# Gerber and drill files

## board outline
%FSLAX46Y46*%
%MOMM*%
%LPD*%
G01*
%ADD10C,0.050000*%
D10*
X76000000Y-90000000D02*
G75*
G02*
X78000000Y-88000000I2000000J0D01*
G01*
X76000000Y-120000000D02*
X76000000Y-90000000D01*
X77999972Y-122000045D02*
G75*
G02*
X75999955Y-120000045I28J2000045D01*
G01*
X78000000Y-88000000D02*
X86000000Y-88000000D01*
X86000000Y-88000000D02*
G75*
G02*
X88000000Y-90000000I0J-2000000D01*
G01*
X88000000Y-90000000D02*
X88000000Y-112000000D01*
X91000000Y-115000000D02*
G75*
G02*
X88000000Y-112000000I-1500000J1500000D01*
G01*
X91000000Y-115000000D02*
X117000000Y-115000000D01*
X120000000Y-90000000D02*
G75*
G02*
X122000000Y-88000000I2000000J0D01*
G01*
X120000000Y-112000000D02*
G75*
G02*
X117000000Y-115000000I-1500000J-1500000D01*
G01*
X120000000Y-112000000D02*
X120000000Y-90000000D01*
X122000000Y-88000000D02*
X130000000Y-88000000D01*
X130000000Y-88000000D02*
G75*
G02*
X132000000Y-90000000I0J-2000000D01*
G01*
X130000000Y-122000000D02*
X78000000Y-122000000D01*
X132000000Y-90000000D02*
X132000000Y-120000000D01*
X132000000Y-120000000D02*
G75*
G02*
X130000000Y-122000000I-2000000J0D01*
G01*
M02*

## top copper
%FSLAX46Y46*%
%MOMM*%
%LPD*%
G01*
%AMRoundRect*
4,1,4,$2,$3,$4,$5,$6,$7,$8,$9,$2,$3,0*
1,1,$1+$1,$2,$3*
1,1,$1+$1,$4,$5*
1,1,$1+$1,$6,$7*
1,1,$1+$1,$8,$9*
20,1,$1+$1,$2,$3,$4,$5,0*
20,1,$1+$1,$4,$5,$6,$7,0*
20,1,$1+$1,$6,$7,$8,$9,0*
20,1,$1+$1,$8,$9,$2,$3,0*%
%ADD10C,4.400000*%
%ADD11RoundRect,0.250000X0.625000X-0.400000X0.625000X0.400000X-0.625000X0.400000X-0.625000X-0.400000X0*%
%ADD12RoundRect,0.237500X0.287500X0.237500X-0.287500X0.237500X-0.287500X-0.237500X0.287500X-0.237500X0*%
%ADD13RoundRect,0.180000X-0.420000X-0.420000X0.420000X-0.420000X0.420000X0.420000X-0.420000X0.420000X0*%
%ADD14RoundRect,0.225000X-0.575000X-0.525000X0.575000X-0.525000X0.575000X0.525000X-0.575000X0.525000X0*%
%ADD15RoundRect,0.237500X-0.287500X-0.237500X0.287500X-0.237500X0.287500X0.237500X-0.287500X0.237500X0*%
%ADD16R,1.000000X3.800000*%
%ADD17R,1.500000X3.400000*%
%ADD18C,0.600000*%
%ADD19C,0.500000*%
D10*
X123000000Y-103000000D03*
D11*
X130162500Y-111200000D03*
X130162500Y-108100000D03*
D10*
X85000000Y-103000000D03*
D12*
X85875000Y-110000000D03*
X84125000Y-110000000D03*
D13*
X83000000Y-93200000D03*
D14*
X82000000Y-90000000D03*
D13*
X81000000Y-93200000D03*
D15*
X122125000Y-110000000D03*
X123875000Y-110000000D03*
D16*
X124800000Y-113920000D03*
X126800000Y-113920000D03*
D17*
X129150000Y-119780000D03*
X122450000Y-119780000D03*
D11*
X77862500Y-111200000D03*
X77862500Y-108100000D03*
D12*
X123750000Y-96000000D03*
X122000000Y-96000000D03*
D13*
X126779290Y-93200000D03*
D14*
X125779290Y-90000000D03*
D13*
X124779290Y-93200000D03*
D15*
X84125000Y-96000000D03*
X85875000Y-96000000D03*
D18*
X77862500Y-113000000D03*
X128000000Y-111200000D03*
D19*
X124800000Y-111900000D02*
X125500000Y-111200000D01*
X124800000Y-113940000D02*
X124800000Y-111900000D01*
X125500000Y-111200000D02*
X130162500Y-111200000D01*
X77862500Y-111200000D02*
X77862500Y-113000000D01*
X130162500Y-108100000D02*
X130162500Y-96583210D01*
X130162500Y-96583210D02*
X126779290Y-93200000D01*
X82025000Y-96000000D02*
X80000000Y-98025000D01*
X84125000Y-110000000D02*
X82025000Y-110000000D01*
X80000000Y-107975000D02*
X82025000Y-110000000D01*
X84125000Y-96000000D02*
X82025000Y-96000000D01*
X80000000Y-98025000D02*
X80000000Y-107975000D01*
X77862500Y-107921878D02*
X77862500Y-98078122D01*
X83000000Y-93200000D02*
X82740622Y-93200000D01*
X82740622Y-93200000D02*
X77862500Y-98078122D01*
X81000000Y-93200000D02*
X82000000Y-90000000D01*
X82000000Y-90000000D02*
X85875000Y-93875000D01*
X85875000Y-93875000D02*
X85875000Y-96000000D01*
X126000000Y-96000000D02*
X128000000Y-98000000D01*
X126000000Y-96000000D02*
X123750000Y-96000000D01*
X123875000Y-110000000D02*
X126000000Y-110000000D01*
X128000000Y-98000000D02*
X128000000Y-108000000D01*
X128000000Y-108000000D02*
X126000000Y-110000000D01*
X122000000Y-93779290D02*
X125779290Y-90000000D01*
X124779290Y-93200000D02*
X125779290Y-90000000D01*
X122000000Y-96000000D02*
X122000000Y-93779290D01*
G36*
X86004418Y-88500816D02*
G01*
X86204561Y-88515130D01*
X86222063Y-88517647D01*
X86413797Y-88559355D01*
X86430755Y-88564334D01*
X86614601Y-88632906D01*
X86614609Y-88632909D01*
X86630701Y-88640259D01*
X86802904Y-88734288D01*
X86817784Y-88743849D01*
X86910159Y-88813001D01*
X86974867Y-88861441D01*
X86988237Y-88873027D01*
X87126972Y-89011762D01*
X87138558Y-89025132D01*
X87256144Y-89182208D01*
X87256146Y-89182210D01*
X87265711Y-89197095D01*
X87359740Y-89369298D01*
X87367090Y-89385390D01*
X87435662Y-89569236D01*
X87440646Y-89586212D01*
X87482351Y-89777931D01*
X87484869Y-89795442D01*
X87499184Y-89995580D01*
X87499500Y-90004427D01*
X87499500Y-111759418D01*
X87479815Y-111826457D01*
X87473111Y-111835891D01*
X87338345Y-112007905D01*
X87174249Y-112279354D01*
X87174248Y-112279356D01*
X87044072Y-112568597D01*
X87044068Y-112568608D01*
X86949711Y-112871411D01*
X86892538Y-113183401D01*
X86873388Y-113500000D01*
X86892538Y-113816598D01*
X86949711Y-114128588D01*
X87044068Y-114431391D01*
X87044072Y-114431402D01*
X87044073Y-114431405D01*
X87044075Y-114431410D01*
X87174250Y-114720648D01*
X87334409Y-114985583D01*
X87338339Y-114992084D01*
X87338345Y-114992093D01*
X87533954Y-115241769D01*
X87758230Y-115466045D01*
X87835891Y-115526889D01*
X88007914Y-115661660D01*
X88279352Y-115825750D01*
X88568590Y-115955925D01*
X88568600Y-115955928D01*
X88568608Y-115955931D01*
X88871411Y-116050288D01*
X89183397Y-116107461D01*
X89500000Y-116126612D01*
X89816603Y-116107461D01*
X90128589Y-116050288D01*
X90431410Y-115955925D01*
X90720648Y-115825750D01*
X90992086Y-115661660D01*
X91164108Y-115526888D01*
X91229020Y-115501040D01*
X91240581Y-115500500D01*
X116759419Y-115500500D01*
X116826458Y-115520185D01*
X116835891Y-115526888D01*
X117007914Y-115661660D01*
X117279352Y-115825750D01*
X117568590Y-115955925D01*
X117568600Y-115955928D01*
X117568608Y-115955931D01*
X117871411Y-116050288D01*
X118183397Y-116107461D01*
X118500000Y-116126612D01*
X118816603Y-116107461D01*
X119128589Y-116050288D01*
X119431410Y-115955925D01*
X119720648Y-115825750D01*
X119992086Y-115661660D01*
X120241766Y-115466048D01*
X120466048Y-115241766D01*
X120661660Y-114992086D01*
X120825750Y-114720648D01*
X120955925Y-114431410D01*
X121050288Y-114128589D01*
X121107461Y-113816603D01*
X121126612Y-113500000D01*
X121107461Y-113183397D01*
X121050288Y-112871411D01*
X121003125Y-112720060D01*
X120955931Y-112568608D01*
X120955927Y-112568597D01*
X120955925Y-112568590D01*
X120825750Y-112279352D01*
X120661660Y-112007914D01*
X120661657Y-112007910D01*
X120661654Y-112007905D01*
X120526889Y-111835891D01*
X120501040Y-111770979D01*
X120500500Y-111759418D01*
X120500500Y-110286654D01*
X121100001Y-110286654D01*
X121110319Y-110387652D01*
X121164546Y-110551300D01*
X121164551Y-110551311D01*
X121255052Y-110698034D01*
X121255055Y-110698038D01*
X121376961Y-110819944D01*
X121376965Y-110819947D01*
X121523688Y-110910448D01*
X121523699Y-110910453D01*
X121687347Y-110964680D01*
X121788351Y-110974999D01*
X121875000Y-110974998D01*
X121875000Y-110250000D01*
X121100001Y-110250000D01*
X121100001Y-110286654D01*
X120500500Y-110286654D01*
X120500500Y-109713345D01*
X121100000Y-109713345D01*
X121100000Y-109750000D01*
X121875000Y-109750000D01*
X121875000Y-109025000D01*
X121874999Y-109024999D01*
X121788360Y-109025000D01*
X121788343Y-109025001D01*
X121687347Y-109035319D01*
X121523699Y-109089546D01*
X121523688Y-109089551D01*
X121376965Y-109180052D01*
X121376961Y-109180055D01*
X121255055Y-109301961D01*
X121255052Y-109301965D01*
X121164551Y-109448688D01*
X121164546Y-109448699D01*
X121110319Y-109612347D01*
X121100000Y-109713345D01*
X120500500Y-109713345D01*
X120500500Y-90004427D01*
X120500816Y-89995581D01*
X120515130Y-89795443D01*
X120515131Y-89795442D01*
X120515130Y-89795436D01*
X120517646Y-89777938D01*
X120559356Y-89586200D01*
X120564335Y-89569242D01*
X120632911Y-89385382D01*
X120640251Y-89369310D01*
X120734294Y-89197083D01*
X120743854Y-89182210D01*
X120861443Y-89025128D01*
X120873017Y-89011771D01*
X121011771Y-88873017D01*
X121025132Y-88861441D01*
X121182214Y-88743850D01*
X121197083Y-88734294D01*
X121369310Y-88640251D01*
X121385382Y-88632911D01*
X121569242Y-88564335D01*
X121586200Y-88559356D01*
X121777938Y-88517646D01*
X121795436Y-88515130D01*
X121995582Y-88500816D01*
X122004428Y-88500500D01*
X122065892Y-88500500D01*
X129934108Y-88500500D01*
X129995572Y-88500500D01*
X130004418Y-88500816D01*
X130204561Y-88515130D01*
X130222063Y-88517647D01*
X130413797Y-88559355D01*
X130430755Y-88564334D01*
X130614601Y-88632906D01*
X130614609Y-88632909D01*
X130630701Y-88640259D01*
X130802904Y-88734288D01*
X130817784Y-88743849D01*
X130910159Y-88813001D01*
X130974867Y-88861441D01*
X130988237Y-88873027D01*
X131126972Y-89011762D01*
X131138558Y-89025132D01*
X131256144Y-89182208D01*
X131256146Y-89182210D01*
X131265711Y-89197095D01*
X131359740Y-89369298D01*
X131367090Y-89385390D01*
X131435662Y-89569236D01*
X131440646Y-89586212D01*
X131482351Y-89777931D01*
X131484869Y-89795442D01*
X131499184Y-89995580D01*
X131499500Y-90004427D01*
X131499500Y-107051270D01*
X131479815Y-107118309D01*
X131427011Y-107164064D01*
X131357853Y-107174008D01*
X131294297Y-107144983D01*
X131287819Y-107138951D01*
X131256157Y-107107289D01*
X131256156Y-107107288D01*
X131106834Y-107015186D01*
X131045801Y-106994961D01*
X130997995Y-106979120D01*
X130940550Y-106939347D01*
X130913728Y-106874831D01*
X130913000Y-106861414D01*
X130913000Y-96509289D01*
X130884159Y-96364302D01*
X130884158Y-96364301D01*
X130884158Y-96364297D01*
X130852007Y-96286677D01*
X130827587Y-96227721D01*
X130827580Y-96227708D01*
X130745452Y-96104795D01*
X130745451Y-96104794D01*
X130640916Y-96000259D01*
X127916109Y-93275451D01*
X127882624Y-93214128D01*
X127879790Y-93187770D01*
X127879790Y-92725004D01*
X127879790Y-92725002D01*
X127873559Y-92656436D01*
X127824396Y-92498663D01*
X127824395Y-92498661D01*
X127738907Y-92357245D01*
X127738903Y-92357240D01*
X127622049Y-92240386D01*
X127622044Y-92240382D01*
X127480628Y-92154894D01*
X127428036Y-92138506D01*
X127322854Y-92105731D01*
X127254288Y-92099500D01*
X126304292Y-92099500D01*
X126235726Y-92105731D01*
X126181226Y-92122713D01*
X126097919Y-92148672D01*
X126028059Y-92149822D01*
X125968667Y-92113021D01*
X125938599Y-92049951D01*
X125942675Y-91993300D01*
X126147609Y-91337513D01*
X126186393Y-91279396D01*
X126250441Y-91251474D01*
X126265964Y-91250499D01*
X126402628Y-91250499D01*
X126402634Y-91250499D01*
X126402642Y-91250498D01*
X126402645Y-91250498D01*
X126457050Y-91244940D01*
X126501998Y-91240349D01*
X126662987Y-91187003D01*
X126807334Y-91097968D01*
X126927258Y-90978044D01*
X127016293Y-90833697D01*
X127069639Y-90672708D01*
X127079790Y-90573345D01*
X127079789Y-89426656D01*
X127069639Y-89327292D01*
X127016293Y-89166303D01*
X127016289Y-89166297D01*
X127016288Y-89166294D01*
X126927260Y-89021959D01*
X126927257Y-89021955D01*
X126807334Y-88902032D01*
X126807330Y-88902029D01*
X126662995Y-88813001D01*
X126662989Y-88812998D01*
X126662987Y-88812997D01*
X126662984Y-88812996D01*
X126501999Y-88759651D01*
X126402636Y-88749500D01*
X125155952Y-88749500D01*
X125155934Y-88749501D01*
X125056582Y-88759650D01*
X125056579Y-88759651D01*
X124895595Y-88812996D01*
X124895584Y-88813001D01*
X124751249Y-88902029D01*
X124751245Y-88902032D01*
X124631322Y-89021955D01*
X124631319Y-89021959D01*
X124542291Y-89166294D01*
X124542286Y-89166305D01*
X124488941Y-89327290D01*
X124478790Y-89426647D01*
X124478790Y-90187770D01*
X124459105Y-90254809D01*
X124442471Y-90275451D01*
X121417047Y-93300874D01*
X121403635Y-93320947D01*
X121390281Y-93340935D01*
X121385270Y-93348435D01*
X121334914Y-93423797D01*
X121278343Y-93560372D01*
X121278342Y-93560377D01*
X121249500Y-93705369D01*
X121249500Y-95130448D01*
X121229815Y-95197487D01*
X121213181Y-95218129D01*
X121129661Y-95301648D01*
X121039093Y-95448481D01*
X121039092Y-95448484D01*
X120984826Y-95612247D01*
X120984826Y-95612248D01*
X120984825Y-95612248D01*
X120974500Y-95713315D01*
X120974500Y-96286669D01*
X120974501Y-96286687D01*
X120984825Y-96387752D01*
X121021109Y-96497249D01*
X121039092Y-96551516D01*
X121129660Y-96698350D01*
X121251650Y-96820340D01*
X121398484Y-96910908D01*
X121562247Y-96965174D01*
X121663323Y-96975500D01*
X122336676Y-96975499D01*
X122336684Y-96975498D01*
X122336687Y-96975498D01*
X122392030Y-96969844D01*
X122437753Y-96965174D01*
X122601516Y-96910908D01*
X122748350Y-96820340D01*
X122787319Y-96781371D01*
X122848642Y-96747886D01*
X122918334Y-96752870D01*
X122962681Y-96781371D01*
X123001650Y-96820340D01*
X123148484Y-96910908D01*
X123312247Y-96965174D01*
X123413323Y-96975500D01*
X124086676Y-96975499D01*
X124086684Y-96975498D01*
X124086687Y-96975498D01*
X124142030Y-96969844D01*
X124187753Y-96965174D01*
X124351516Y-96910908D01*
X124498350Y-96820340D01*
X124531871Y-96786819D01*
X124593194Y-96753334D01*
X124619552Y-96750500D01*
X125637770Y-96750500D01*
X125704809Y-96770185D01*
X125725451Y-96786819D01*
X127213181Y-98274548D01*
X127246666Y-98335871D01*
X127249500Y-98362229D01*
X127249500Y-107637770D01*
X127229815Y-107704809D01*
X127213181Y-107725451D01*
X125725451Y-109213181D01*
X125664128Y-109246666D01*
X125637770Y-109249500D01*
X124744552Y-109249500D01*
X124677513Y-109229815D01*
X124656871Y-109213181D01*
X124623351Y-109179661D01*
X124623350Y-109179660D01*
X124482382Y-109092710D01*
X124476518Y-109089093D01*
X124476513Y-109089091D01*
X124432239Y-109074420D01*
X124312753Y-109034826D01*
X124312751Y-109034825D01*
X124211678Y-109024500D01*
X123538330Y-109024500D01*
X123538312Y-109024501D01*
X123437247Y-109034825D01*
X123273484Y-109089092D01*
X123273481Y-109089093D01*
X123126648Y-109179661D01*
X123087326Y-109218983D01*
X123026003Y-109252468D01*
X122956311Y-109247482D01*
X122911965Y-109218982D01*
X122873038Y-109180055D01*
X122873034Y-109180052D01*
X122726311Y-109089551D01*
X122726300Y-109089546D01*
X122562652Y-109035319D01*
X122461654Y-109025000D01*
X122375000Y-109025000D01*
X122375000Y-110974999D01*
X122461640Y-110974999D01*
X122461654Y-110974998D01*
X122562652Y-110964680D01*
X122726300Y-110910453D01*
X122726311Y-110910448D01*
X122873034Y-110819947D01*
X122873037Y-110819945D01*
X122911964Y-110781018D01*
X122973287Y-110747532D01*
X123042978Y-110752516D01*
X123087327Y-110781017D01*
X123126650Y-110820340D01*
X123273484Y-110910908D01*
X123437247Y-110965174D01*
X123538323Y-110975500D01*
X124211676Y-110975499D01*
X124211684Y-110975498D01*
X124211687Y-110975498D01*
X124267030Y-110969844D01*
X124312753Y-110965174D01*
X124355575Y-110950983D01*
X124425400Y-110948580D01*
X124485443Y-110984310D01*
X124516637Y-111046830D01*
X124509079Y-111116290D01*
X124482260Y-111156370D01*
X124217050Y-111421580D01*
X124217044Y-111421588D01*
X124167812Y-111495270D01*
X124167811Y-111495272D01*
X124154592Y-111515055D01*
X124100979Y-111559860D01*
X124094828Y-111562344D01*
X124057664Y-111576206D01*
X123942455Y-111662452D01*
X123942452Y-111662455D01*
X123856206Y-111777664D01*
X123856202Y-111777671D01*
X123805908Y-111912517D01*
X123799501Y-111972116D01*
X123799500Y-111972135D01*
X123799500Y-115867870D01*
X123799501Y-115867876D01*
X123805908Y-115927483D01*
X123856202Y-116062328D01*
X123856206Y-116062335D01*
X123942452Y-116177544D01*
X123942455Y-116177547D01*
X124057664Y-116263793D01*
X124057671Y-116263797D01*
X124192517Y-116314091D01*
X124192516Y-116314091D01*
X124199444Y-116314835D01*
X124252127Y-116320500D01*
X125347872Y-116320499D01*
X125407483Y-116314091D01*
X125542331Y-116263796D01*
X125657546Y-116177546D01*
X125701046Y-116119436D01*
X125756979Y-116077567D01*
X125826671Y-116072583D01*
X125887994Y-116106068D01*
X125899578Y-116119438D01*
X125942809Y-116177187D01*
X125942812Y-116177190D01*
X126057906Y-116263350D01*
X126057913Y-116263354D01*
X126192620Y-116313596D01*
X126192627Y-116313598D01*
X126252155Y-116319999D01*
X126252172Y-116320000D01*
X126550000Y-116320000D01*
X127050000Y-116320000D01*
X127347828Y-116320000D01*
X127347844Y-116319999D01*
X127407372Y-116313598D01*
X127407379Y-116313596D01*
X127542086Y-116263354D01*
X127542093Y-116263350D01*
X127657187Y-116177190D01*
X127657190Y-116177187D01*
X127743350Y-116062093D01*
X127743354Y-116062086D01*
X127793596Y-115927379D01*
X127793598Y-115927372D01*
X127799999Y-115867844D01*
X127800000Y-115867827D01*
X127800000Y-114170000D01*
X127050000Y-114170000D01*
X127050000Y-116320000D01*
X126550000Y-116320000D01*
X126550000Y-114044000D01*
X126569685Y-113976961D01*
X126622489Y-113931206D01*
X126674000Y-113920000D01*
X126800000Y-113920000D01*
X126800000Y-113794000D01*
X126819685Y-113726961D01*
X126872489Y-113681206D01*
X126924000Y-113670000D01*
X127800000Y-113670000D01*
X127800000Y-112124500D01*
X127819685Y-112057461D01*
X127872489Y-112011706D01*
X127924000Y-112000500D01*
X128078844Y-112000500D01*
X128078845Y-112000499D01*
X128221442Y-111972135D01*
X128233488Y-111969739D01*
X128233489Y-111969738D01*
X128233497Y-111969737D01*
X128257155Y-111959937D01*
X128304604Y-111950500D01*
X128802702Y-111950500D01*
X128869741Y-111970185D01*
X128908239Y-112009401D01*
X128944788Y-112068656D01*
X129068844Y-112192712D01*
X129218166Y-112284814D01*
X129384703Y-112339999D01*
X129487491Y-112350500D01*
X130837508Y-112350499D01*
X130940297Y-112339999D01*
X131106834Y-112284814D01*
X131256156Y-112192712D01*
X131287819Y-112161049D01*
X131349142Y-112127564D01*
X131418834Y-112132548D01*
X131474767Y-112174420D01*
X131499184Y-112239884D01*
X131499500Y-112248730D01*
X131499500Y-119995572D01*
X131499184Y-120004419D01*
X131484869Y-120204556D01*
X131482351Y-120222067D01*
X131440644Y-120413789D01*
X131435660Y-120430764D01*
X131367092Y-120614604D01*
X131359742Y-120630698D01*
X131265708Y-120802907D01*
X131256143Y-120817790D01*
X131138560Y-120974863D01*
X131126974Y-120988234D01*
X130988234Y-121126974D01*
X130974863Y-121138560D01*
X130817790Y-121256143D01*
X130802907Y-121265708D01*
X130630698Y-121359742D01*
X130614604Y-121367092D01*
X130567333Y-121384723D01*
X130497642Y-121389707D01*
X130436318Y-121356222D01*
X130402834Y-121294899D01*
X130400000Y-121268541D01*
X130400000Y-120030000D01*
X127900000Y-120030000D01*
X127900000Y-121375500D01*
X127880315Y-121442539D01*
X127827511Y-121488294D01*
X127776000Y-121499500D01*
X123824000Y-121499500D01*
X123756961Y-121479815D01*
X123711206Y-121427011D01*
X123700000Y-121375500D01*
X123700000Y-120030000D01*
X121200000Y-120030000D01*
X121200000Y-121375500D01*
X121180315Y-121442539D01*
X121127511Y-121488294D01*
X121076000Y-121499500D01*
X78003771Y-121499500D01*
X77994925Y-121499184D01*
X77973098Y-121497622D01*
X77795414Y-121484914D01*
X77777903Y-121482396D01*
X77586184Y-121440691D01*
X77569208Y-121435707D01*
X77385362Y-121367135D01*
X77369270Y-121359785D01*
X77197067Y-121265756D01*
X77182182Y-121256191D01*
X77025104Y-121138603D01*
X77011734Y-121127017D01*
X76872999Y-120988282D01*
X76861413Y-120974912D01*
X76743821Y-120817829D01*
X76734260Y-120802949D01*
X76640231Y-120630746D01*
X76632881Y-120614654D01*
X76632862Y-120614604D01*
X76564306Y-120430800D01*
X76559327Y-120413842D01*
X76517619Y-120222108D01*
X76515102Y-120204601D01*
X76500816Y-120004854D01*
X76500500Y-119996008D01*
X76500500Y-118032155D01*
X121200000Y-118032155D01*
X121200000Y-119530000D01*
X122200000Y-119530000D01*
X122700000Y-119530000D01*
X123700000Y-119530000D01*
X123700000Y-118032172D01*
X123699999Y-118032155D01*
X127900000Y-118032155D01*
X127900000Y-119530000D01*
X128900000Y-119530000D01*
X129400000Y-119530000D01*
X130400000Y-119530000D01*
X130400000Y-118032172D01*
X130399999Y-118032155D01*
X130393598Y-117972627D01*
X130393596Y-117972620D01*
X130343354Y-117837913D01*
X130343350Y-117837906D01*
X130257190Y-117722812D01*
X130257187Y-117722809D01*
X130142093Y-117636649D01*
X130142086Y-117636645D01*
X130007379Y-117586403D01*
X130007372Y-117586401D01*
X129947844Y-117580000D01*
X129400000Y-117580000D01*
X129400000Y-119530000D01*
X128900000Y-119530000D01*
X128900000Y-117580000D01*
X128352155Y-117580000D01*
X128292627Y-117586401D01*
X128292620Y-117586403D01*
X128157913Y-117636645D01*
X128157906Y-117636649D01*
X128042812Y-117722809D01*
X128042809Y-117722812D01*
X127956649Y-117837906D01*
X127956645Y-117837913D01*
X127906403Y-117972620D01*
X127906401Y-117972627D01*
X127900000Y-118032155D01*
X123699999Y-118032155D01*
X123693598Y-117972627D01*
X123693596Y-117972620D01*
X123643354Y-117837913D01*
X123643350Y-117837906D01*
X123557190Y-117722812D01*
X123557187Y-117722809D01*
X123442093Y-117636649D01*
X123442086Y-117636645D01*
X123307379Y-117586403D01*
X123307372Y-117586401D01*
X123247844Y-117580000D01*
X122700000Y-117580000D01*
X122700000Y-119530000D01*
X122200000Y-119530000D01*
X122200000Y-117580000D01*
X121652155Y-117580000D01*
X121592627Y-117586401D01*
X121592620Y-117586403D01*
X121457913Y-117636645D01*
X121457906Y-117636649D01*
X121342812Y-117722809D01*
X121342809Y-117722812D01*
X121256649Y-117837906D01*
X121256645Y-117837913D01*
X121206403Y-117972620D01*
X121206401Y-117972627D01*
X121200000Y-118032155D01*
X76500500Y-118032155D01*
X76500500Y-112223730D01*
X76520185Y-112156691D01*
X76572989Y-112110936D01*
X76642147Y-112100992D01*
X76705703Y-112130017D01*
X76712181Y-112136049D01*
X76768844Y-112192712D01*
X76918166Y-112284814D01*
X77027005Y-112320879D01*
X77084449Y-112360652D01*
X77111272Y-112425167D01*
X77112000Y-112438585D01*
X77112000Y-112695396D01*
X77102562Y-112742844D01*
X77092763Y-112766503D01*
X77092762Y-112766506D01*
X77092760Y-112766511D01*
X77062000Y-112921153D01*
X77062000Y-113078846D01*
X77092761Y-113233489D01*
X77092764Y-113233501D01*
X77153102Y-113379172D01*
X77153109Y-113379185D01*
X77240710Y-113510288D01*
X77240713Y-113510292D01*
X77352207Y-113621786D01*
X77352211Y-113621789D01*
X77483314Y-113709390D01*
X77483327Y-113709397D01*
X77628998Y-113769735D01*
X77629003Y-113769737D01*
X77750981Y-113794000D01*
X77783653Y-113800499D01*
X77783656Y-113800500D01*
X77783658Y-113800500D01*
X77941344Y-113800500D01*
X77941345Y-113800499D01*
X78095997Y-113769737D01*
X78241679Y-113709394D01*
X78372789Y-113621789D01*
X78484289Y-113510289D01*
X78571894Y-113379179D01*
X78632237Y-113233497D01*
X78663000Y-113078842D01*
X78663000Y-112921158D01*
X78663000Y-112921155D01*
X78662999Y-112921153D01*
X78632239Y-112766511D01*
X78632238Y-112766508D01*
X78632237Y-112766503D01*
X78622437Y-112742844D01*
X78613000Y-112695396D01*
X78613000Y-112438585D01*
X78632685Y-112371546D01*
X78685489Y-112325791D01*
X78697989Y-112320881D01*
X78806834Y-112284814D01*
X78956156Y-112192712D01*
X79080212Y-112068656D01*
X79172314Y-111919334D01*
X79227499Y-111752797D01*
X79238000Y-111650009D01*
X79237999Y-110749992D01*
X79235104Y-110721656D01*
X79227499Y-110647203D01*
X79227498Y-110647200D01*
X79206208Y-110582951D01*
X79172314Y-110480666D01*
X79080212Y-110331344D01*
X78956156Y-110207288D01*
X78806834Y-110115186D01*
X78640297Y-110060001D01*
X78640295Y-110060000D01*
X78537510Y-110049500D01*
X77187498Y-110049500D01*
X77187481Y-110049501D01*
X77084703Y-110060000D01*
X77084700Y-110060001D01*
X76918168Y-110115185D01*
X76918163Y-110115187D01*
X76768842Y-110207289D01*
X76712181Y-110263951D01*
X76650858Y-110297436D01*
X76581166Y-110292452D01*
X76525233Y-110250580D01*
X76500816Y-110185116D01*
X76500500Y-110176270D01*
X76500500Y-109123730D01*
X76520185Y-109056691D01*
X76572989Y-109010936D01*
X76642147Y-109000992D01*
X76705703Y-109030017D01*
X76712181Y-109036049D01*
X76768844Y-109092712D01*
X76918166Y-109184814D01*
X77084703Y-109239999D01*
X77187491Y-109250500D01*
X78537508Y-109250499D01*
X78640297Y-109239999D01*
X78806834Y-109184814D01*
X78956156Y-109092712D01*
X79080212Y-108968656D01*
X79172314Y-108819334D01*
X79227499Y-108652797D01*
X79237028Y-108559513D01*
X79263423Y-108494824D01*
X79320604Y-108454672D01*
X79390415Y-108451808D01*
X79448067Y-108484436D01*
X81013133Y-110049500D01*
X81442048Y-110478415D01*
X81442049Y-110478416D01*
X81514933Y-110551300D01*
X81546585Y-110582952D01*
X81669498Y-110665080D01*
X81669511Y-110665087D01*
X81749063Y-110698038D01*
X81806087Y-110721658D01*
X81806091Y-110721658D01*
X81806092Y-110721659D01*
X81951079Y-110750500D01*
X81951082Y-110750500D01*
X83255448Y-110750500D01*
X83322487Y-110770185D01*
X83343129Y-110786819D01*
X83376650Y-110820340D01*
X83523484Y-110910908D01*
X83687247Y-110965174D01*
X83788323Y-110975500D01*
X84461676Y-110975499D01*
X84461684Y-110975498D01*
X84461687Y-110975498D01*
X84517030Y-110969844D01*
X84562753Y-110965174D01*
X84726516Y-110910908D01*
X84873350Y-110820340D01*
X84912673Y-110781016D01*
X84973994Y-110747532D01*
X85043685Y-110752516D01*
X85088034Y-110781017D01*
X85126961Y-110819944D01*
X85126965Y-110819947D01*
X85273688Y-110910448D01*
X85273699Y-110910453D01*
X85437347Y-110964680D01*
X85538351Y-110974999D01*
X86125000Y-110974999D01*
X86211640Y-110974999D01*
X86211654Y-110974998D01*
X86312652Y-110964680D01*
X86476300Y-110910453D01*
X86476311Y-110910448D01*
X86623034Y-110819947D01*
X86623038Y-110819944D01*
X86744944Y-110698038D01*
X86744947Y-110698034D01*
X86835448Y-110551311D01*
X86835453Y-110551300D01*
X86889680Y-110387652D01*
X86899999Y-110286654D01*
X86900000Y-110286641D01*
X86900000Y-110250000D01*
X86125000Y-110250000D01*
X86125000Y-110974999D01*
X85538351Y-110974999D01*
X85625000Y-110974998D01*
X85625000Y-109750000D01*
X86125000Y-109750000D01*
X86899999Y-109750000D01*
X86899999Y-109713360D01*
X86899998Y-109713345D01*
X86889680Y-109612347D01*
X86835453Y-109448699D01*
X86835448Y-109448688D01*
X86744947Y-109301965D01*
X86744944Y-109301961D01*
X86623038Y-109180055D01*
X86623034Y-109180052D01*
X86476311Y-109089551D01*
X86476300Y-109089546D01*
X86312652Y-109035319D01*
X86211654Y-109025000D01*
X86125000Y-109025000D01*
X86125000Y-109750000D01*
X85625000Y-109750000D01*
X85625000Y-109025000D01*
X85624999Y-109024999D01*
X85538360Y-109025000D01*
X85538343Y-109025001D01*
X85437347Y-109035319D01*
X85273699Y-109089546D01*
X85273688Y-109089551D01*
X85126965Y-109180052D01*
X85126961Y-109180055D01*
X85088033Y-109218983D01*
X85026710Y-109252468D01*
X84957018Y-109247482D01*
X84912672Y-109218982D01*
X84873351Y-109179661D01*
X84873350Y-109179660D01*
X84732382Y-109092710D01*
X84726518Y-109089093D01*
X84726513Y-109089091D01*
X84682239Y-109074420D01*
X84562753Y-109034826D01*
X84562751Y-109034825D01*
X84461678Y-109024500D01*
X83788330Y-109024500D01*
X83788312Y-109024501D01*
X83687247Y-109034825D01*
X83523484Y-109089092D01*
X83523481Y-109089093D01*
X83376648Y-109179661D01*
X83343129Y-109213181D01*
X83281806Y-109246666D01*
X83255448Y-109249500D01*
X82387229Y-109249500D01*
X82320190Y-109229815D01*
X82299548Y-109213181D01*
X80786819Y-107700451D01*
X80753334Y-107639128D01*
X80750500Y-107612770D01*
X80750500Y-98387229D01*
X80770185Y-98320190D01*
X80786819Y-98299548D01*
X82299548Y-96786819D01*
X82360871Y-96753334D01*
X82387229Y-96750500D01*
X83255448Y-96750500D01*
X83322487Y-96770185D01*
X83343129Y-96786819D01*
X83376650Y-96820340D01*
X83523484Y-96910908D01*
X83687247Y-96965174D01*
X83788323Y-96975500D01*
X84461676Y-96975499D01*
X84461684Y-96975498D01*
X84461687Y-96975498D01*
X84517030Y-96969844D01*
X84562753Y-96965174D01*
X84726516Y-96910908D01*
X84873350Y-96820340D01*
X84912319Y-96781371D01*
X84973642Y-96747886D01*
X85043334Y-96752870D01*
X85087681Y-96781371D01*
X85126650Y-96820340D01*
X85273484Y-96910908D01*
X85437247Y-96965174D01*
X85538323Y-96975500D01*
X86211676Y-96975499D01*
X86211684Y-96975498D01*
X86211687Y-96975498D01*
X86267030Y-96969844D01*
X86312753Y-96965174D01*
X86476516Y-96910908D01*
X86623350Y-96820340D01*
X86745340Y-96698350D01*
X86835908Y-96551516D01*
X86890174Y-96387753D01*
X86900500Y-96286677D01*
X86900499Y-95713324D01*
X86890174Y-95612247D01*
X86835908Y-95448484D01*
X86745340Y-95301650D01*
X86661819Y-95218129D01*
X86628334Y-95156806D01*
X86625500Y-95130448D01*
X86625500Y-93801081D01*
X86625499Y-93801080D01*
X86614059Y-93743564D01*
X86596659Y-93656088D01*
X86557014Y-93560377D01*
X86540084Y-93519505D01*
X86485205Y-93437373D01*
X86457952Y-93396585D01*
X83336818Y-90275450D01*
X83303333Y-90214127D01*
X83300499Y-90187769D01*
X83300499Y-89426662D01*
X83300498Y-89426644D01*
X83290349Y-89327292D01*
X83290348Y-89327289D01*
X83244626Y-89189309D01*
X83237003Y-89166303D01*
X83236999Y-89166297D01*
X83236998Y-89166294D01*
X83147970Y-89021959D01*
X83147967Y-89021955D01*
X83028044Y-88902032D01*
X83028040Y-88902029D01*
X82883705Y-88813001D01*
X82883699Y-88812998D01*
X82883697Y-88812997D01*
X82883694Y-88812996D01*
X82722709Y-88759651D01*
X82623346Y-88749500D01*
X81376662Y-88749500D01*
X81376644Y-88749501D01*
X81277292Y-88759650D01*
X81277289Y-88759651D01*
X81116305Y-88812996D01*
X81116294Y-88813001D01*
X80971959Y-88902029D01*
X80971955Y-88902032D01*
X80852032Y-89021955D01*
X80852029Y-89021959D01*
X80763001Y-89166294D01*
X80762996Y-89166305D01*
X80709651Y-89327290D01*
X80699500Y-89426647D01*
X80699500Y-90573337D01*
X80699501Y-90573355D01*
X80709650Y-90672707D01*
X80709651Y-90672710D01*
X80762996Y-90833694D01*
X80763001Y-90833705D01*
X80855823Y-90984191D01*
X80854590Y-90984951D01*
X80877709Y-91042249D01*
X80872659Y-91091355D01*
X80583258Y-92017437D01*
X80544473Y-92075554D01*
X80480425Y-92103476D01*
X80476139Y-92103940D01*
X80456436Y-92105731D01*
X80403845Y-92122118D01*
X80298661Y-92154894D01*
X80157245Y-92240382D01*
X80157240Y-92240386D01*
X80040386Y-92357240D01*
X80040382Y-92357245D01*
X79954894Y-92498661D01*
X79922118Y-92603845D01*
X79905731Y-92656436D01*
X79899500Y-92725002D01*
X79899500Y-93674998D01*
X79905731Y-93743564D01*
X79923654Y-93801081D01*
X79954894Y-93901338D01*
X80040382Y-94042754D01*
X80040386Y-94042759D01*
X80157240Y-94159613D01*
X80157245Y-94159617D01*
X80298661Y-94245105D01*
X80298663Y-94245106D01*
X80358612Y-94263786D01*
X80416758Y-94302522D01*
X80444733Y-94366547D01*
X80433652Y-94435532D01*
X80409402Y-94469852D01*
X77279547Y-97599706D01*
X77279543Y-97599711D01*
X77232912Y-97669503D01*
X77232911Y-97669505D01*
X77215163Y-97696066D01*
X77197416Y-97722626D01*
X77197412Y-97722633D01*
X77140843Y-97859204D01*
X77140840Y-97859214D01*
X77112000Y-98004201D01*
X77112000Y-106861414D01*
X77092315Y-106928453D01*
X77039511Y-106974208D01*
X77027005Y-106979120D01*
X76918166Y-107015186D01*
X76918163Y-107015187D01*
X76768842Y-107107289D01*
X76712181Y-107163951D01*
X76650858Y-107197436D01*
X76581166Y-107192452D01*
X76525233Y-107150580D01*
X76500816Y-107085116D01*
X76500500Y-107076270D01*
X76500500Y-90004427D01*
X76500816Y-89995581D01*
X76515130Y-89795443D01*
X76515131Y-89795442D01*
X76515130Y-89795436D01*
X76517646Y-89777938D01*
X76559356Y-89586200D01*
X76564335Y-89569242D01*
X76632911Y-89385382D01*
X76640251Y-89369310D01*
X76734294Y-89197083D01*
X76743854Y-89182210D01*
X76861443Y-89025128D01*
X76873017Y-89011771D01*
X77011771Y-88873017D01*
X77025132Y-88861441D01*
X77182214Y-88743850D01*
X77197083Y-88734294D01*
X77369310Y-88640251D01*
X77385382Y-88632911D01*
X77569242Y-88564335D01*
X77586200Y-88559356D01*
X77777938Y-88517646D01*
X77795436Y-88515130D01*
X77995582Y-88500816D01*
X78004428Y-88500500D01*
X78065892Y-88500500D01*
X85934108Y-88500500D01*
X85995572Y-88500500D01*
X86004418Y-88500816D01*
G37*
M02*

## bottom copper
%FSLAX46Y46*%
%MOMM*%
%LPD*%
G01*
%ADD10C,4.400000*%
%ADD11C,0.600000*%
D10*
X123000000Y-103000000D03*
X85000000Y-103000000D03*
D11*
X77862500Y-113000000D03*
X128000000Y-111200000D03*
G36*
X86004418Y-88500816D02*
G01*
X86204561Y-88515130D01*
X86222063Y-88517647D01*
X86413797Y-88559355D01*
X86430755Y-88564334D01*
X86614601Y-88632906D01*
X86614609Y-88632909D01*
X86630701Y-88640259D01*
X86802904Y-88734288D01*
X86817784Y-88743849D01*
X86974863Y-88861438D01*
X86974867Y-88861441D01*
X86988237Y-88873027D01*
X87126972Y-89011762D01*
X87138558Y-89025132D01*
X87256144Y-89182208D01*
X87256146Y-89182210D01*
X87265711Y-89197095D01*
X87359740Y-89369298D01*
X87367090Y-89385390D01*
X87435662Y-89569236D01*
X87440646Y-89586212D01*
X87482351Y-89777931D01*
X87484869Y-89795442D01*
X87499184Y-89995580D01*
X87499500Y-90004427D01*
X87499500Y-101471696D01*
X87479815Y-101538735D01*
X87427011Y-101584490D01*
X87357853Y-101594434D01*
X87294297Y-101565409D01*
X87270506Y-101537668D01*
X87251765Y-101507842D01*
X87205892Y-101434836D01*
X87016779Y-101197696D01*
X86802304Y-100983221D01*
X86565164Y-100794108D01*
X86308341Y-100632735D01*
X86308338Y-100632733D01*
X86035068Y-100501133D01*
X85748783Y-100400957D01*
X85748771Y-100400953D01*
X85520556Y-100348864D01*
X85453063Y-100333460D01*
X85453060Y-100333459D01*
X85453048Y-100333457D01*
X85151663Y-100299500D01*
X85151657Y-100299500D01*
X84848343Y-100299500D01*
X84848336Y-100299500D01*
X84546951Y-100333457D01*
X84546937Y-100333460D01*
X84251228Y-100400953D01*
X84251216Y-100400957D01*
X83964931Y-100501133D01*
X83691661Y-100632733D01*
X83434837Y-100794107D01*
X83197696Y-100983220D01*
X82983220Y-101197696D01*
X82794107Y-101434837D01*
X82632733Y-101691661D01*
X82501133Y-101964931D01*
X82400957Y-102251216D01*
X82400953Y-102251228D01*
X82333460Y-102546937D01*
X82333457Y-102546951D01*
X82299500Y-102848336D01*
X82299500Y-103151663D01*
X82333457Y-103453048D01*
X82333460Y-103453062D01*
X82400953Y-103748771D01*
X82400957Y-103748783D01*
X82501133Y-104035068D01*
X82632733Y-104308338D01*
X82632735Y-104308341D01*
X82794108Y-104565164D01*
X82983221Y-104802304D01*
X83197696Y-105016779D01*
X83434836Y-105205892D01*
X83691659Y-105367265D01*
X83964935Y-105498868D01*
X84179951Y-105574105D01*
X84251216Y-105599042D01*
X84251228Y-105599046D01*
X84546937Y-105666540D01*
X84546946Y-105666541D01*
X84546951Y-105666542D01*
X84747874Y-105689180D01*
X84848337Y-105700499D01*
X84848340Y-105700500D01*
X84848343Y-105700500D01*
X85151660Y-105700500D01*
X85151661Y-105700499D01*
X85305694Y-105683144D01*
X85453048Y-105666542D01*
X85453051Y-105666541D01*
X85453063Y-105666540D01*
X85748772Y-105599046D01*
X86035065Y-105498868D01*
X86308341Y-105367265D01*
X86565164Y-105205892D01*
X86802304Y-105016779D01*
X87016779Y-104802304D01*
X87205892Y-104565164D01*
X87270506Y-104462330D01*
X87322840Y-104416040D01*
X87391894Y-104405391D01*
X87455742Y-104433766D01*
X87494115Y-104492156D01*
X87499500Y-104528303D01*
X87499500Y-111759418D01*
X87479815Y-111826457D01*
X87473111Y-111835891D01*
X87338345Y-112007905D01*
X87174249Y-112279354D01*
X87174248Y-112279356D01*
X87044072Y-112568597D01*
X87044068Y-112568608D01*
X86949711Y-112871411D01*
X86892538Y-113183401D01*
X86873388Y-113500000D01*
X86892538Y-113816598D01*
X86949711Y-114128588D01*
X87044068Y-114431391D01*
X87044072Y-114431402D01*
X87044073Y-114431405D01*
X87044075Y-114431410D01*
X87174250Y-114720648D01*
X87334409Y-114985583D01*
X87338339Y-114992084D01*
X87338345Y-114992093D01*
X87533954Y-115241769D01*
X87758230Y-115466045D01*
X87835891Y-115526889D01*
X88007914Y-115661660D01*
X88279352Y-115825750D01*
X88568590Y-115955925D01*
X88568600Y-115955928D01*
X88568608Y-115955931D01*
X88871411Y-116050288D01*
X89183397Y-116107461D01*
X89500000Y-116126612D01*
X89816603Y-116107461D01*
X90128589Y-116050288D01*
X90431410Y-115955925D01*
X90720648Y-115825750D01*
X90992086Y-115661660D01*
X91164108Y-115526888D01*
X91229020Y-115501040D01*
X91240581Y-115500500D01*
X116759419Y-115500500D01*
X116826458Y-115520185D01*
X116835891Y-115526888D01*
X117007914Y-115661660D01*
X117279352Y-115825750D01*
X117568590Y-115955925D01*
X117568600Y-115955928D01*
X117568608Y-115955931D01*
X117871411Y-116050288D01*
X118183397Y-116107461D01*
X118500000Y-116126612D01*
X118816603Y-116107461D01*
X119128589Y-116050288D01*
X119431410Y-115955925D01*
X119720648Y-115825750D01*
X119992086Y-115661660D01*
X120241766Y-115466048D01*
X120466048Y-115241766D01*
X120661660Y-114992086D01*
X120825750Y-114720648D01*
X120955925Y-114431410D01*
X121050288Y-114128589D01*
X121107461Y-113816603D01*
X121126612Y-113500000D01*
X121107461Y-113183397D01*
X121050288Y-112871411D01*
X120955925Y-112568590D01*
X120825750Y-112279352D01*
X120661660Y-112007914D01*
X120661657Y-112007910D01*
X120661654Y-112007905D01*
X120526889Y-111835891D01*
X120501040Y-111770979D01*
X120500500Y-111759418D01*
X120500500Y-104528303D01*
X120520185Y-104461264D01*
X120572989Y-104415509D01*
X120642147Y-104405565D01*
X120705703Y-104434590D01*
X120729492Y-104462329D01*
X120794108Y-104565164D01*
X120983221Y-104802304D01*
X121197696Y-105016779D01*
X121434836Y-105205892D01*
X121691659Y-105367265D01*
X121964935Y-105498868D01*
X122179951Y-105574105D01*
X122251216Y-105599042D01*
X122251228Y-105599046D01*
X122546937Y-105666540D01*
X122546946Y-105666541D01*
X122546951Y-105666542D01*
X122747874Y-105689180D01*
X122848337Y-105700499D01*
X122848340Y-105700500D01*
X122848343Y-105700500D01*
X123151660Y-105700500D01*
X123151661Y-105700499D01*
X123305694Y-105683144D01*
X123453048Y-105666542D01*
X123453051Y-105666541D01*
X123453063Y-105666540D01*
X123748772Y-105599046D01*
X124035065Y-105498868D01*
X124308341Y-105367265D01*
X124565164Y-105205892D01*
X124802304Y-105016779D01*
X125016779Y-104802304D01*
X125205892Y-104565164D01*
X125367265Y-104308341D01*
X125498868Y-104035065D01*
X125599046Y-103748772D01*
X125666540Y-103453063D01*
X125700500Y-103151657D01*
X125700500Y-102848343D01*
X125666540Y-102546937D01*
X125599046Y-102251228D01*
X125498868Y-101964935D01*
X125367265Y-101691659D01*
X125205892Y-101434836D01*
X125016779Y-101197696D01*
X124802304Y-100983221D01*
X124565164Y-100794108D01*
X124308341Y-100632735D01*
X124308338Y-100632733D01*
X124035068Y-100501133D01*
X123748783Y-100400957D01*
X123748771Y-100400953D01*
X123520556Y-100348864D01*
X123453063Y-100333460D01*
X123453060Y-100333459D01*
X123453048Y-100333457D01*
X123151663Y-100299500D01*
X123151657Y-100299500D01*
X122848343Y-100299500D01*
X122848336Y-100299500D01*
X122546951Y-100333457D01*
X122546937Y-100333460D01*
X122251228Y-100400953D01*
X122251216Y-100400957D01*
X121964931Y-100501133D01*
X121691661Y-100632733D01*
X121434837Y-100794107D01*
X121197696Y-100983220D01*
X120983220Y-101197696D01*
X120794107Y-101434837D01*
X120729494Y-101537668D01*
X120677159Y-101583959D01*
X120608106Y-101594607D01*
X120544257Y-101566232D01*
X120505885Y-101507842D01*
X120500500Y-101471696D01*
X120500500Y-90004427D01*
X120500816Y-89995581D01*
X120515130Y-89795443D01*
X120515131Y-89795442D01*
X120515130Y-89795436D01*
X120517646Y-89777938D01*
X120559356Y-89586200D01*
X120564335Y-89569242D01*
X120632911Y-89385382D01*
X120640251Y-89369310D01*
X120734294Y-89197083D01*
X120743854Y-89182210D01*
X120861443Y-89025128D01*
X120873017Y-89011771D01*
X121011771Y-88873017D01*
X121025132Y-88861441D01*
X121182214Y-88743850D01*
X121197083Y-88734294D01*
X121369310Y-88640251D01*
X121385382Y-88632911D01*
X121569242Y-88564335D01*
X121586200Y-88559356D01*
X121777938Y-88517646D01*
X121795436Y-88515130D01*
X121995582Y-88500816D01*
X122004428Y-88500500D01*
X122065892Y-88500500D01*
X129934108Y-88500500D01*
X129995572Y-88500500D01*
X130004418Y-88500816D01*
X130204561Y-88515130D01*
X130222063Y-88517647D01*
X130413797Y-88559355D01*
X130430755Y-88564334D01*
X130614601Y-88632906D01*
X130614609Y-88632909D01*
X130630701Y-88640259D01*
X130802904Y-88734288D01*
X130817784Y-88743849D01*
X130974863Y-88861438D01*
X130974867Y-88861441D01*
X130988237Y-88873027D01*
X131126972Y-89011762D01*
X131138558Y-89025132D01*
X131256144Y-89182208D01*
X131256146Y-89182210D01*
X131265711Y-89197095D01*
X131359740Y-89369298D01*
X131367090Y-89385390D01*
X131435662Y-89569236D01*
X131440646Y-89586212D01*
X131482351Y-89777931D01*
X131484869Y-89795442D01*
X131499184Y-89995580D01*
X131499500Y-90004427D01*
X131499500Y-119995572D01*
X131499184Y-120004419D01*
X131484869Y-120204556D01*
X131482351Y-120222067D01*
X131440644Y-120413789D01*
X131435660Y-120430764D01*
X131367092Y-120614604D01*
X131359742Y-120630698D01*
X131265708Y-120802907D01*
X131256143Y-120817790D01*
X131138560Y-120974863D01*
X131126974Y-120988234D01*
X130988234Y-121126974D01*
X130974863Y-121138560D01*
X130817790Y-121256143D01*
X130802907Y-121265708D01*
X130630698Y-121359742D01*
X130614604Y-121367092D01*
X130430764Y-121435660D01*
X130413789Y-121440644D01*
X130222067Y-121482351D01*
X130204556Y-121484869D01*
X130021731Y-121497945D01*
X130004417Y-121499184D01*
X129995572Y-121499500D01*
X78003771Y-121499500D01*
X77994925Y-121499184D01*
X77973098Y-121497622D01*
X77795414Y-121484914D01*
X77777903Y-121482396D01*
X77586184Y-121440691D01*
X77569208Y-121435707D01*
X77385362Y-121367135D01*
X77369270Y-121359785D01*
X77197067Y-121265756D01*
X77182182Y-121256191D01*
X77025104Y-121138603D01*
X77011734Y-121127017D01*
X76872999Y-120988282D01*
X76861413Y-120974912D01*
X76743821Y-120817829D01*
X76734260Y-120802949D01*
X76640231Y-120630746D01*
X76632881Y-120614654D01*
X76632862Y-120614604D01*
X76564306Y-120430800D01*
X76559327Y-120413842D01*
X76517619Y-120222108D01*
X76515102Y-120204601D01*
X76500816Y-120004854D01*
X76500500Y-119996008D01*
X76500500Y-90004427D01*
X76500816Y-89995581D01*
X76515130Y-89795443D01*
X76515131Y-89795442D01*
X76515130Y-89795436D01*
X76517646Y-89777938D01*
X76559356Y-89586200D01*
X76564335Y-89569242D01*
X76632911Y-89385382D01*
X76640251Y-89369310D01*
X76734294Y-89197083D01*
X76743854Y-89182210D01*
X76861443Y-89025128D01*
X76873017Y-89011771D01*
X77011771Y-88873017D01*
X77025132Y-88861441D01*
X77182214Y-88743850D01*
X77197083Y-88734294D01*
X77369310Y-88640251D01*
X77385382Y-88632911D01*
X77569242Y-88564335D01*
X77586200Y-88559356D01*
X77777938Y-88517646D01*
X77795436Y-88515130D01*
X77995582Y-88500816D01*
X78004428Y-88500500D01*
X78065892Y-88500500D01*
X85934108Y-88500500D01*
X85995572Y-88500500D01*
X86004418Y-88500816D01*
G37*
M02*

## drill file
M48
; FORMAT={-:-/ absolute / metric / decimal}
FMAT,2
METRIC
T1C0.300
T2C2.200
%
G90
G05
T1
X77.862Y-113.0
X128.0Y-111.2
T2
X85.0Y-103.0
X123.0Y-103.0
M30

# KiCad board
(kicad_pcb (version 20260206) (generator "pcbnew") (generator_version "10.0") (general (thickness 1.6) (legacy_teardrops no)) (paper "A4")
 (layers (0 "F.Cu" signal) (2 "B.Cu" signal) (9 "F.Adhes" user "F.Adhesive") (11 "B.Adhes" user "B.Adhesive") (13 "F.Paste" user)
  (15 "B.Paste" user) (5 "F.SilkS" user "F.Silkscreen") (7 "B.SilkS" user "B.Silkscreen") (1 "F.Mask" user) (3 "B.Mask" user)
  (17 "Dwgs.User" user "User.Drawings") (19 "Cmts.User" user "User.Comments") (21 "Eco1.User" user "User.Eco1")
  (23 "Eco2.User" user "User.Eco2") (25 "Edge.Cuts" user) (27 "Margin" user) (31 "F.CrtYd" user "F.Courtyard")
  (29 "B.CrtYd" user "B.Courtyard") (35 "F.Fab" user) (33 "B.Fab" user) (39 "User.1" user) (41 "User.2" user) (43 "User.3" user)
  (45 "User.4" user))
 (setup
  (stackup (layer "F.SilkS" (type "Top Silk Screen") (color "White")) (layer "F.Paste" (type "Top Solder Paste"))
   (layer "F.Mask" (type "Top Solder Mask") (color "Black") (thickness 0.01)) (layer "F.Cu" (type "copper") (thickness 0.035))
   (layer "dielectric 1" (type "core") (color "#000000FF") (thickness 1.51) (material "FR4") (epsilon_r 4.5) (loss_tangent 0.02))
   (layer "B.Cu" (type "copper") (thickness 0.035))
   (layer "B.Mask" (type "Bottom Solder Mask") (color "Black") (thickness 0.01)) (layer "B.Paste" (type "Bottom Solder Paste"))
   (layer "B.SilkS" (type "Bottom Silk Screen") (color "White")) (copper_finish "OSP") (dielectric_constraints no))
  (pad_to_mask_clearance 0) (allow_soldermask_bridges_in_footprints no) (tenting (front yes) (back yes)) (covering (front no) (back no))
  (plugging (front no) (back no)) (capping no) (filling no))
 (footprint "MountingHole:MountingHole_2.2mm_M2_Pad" (layer "F.Cu") (at 123 103)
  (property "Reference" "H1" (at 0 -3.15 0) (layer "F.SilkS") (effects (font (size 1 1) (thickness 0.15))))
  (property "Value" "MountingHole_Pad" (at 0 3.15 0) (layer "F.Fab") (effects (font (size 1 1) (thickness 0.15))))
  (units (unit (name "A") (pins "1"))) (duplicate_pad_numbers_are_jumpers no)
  (pad "1" thru_hole circle (at 0 0) (size 4.4 4.4) (drill 2.2) (layers "*.Cu" "*.Mask") (remove_unused_layers no) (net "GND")
   (zone_connect 2)))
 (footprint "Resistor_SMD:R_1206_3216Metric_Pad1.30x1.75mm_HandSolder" (layer "F.Cu") (at 130.1625 109.65 90)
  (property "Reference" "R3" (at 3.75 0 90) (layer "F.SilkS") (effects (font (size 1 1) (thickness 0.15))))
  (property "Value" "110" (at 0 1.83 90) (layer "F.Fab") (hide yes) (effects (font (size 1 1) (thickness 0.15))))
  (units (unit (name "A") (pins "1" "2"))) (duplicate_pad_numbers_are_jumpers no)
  (pad "1" smd roundrect (at -1.55 0 90) (size 1.3 1.75) (layers "F.Cu" "F.Mask" "F.Paste") (roundrect_rratio 0.192308) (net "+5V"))
  (pad "2" smd roundrect (at 1.55 0 90) (size 1.3 1.75) (layers "F.Cu" "F.Mask" "F.Paste") (roundrect_rratio 0.192308) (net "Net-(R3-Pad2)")))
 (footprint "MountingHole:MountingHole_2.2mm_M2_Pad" (layer "F.Cu") (at 85 103)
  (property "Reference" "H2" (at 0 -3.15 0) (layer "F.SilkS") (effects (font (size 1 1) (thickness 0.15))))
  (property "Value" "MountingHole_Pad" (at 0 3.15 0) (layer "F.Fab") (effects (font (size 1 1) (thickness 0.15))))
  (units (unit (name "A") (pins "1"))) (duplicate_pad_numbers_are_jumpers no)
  (pad "1" thru_hole circle (at 0 0) (size 4.4 4.4) (drill 2.2) (layers "*.Cu" "*.Mask") (remove_unused_layers no) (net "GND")
   (zone_connect 2)))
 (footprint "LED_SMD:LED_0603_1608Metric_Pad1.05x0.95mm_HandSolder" (layer "F.Cu") (at 85 110 180)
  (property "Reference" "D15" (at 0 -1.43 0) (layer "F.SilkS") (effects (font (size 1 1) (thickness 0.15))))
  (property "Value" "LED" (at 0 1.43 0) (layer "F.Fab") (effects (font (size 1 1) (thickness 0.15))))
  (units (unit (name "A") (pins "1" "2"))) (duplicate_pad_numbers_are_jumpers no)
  (pad "1" smd roundrect (at -0.875 0 180) (size 1.05 0.95) (layers "F.Cu" "F.Mask" "F.Paste") (roundrect_rratio 0.25) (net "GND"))
  (pad "2" smd roundrect (at 0.875 0 180) (size 1.05 0.95) (layers "F.Cu" "F.Mask" "F.Paste") (roundrect_rratio 0.25) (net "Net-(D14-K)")))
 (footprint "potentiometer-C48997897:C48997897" (layer "F.Cu") (at 82 95.4)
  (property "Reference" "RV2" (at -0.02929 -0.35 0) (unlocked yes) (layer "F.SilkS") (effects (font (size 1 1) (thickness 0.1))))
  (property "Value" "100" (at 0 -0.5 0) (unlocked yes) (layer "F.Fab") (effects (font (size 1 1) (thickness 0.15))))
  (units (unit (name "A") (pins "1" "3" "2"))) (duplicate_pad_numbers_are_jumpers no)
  (pad "1" smd roundrect (at 1 -2.2) (size 1.2 1.2) (layers "F.Cu" "F.Mask" "F.Paste") (roundrect_rratio 0.15) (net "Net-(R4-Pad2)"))
  (pad "2" smd roundrect (at 0 -5.4) (size 1.6 1.5) (layers "F.Cu" "F.Mask" "F.Paste") (roundrect_rratio 0.15) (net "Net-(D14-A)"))
  (pad "3" smd roundrect (at -1 -2.2) (size 1.2 1.2) (layers "F.Cu" "F.Mask" "F.Paste") (roundrect_rratio 0.15) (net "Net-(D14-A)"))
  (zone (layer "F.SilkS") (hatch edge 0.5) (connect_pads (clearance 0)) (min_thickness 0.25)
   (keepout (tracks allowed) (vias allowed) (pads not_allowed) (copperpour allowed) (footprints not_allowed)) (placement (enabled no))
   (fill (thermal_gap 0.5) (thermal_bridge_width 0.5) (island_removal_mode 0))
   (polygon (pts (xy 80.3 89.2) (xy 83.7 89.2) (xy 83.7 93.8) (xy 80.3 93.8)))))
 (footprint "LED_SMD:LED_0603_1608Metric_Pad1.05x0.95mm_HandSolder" (layer "F.Cu") (at 123 110)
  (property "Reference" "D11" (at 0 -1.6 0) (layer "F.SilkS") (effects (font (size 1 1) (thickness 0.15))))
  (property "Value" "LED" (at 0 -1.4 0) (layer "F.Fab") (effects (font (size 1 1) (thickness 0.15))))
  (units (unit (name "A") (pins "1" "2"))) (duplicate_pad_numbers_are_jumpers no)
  (pad "1" smd roundrect (at -0.875 0) (size 1.05 0.95) (layers "F.Cu" "F.Mask" "F.Paste") (roundrect_rratio 0.25) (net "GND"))
  (pad "2" smd roundrect (at 0.875 0) (size 1.05 0.95) (layers "F.Cu" "F.Mask" "F.Paste") (roundrect_rratio 0.25) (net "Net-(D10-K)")))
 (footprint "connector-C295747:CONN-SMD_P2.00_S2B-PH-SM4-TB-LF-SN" (layer "F.Cu") (at 125.8 116.85)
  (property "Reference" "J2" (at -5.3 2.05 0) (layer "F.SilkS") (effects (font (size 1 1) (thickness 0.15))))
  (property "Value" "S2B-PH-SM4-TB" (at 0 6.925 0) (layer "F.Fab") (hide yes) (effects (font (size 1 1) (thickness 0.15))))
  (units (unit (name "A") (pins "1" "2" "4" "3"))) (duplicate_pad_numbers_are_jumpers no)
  (pad "1" smd rect (at -1 -2.93) (size 1 3.8) (layers "F.Cu" "F.Mask" "F.Paste") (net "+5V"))
  (pad "2" smd rect (at 1 -2.93) (size 1 3.8) (layers "F.Cu" "F.Mask" "F.Paste") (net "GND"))
  (pad "3" smd rect (at 3.35 2.93) (size 1.5 3.4) (layers "F.Cu" "F.Mask" "F.Paste") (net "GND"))
  (pad "4" smd rect (at -3.35 2.93) (size 1.5 3.4) (layers "F.Cu" "F.Mask" "F.Paste") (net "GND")))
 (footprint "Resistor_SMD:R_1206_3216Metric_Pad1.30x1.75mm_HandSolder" (layer "F.Cu") (at 77.8625 109.65 90)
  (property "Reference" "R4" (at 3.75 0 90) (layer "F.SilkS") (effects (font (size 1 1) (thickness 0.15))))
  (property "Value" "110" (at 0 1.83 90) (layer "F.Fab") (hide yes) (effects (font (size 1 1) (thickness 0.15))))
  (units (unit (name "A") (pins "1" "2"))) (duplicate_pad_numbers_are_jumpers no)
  (pad "1" smd roundrect (at -1.55 0 90) (size 1.3 1.75) (layers "F.Cu" "F.Mask" "F.Paste") (roundrect_rratio 0.192308) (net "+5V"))
  (pad "2" smd roundrect (at 1.55 0 90) (size 1.3 1.75) (layers "F.Cu" "F.Mask" "F.Paste") (roundrect_rratio 0.192308) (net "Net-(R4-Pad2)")))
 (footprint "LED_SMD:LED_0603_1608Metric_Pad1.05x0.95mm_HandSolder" (layer "F.Cu") (at 122.875 96 180)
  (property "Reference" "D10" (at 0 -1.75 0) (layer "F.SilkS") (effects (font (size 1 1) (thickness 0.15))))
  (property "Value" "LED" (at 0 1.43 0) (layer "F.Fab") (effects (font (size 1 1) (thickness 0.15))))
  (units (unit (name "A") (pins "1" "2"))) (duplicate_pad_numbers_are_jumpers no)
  (pad "1" smd roundrect (at -0.875 0 180) (size 1.05 0.95) (layers "F.Cu" "F.Mask" "F.Paste") (roundrect_rratio 0.25) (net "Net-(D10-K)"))
  (pad "2" smd roundrect (at 0.875 0 180) (size 1.05 0.95) (layers "F.Cu" "F.Mask" "F.Paste") (roundrect_rratio 0.25) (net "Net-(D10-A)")))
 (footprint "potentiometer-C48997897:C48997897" (layer "F.Cu") (at 125.77929 95.4)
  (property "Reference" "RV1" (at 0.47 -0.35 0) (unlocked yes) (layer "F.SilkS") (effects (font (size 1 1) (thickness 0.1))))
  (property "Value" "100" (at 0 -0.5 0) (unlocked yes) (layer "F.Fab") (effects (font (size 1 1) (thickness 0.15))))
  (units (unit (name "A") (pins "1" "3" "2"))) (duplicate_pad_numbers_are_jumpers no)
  (pad "1" smd roundrect (at 1 -2.2) (size 1.2 1.2) (layers "F.Cu" "F.Mask" "F.Paste") (roundrect_rratio 0.15) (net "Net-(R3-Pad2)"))
  (pad "2" smd roundrect (at 0 -5.4) (size 1.6 1.5) (layers "F.Cu" "F.Mask" "F.Paste") (roundrect_rratio 0.15) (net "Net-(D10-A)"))
  (pad "3" smd roundrect (at -1 -2.2) (size 1.2 1.2) (layers "F.Cu" "F.Mask" "F.Paste") (roundrect_rratio 0.15) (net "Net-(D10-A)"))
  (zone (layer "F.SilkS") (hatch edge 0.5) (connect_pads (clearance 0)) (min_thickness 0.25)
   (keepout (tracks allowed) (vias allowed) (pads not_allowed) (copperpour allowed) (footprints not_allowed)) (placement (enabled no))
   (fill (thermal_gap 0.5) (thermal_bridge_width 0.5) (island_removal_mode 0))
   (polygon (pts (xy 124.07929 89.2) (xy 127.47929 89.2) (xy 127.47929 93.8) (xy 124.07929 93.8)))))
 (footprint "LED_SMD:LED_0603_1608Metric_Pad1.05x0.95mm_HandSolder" (layer "F.Cu") (at 85 96)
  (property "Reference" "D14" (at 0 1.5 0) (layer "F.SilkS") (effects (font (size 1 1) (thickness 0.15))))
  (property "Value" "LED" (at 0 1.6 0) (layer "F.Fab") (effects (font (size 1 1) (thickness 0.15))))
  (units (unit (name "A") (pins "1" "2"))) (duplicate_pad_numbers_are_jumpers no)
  (pad "1" smd roundrect (at -0.875 0) (size 1.05 0.95) (layers "F.Cu" "F.Mask" "F.Paste") (roundrect_rratio 0.25) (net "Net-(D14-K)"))
  (pad "2" smd roundrect (at 0.875 0) (size 1.05 0.95) (layers "F.Cu" "F.Mask" "F.Paste") (roundrect_rratio 0.25) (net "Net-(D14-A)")))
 (gr_arc (start 76 90) (mid 76.585786 88.585786) (end 78 88) (stroke (width 0.05) (type default)) (layer "Edge.Cuts"))
 (gr_line (start 76 120) (end 76 90) (stroke (width 0.05) (type default)) (layer "Edge.Cuts"))
 (gr_arc (start 77.999972 122.000045) (mid 76.585758 121.414258) (end 75.999972 120.000045) (stroke (width 0.05) (type default))
  (layer "Edge.Cuts"))
 (gr_line (start 78 88) (end 86 88) (stroke (width 0.05) (type default)) (layer "Edge.Cuts"))
 (gr_arc (start 86 88) (mid 87.414213 88.585786) (end 88 90) (stroke (width 0.05) (type default)) (layer "Edge.Cuts"))
 (gr_line (start 88 90) (end 88 112) (stroke (width 0.05) (type default)) (layer "Edge.Cuts"))
 (gr_arc (start 91 115) (mid 88 115) (end 88 112) (stroke (width 0.05) (type default)) (layer "Edge.Cuts"))
 (gr_line (start 91 115) (end 117 115) (stroke (width 0.05) (type default)) (layer "Edge.Cuts"))
 (gr_arc (start 120 90) (mid 120.585786 88.585786) (end 122 88) (stroke (width 0.05) (type default)) (layer "Edge.Cuts"))
 (gr_arc (start 120 112) (mid 120 115) (end 117 115) (stroke (width 0.05) (type default)) (layer "Edge.Cuts"))
 (gr_line (start 120 112) (end 120 90) (stroke (width 0.05) (type default)) (layer "Edge.Cuts"))
 (gr_line (start 122 88) (end 130 88) (stroke (width 0.05) (type default)) (layer "Edge.Cuts"))
 (gr_arc (start 130 88) (mid 131.414213 88.585786) (end 132 90) (stroke (width 0.05) (type default)) (layer "Edge.Cuts"))
 (gr_line (start 130 122) (end 78 122) (stroke (width 0.05) (type default)) (layer "Edge.Cuts"))
 (gr_line (start 132 90) (end 132 120) (stroke (width 0.05) (type default)) (layer "Edge.Cuts"))
 (gr_arc (start 132 120) (mid 131.414213 121.414213) (end 130 122) (stroke (width 0.05) (type default)) (layer "Edge.Cuts"))
 (segment (start 124.8 111.9) (end 125.5 111.2) (width 0.5) (layer "F.Cu") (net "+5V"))
 (segment (start 124.8 113.94) (end 124.8 111.9) (width 0.5) (layer "F.Cu") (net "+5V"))
 (segment (start 125.5 111.2) (end 130.1625 111.2) (width 0.5) (layer "F.Cu") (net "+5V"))
 (segment (start 77.8625 111.2) (end 77.8625 113) (width 0.5) (layer "F.Cu") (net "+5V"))
 (via (at 77.8625 113) (size 0.6) (drill 0.3) (layers "F.Cu" "B.Cu") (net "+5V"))
 (via (at 128 111.2) (size 0.6) (drill 0.3) (layers "F.Cu" "B.Cu") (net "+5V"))
 (segment (start 130.1625 108.1) (end 130.1625 96.58321) (width 0.5) (layer "F.Cu") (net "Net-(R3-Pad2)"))
 (segment (start 130.1625 96.58321) (end 126.77929 93.2) (width 0.5) (layer "F.Cu") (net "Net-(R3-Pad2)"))
 (segment (start 82.025 96) (end 80 98.025) (width 0.5) (layer "F.Cu") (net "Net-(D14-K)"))
 (segment (start 84.125 110) (end 82.025 110) (width 0.5) (layer "F.Cu") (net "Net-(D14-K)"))
 (segment (start 80 107.975) (end 82.025 110) (width 0.5) (layer "F.Cu") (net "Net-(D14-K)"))
 (segment (start 84.125 96) (end 82.025 96) (width 0.5) (layer "F.Cu") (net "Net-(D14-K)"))
 (segment (start 80 98.025) (end 80 107.975) (width 0.5) (layer "F.Cu") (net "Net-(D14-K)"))
 (segment (start 77.8625 107.921878) (end 77.8625 98.078122) (width 0.5) (layer "F.Cu") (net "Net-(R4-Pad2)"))
 (segment (start 83 93.2) (end 82.740622 93.2) (width 0.5) (layer "F.Cu") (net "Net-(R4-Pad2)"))
 (segment (start 82.740622 93.2) (end 77.8625 98.078122) (width 0.5) (layer "F.Cu") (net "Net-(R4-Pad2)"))
 (segment (start 81 93.2) (end 82 90) (width 0.5) (layer "F.Cu") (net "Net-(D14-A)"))
 (segment (start 82 90) (end 85.875 93.875) (width 0.5) (layer "F.Cu") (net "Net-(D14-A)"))
 (segment (start 85.875 93.875) (end 85.875 96) (width 0.5) (layer "F.Cu") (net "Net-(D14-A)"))
 (segment (start 126 96) (end 128 98) (width 0.5) (layer "F.Cu") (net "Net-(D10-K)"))
 (segment (start 126 96) (end 123.75 96) (width 0.5) (layer "F.Cu") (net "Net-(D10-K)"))
 (segment (start 123.875 110) (end 126 110) (width 0.5) (layer "F.Cu") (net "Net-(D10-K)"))
 (segment (start 128 98) (end 128 108) (width 0.5) (layer "F.Cu") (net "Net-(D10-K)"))
 (segment (start 128 108) (end 126 110) (width 0.5) (layer "F.Cu") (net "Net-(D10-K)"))
 (segment (start 122 93.77929) (end 125.77929 90) (width 0.5) (layer "F.Cu") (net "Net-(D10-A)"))
 (segment (start 124.77929 93.2) (end 125.77929 90) (width 0.5) (layer "F.Cu") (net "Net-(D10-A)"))
 (segment (start 122 96) (end 122 93.77929) (width 0.5) (layer "F.Cu") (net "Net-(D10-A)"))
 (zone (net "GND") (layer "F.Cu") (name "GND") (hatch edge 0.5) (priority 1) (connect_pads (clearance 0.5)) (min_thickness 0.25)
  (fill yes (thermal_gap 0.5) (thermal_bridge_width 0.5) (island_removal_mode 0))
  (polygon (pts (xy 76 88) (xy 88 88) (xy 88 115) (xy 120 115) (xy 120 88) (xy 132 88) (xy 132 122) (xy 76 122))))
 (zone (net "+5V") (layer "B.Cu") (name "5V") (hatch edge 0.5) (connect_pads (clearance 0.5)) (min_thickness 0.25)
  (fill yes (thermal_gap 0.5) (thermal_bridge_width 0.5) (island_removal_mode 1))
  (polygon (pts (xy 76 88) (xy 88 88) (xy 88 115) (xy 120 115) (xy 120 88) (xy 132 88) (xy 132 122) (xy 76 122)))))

